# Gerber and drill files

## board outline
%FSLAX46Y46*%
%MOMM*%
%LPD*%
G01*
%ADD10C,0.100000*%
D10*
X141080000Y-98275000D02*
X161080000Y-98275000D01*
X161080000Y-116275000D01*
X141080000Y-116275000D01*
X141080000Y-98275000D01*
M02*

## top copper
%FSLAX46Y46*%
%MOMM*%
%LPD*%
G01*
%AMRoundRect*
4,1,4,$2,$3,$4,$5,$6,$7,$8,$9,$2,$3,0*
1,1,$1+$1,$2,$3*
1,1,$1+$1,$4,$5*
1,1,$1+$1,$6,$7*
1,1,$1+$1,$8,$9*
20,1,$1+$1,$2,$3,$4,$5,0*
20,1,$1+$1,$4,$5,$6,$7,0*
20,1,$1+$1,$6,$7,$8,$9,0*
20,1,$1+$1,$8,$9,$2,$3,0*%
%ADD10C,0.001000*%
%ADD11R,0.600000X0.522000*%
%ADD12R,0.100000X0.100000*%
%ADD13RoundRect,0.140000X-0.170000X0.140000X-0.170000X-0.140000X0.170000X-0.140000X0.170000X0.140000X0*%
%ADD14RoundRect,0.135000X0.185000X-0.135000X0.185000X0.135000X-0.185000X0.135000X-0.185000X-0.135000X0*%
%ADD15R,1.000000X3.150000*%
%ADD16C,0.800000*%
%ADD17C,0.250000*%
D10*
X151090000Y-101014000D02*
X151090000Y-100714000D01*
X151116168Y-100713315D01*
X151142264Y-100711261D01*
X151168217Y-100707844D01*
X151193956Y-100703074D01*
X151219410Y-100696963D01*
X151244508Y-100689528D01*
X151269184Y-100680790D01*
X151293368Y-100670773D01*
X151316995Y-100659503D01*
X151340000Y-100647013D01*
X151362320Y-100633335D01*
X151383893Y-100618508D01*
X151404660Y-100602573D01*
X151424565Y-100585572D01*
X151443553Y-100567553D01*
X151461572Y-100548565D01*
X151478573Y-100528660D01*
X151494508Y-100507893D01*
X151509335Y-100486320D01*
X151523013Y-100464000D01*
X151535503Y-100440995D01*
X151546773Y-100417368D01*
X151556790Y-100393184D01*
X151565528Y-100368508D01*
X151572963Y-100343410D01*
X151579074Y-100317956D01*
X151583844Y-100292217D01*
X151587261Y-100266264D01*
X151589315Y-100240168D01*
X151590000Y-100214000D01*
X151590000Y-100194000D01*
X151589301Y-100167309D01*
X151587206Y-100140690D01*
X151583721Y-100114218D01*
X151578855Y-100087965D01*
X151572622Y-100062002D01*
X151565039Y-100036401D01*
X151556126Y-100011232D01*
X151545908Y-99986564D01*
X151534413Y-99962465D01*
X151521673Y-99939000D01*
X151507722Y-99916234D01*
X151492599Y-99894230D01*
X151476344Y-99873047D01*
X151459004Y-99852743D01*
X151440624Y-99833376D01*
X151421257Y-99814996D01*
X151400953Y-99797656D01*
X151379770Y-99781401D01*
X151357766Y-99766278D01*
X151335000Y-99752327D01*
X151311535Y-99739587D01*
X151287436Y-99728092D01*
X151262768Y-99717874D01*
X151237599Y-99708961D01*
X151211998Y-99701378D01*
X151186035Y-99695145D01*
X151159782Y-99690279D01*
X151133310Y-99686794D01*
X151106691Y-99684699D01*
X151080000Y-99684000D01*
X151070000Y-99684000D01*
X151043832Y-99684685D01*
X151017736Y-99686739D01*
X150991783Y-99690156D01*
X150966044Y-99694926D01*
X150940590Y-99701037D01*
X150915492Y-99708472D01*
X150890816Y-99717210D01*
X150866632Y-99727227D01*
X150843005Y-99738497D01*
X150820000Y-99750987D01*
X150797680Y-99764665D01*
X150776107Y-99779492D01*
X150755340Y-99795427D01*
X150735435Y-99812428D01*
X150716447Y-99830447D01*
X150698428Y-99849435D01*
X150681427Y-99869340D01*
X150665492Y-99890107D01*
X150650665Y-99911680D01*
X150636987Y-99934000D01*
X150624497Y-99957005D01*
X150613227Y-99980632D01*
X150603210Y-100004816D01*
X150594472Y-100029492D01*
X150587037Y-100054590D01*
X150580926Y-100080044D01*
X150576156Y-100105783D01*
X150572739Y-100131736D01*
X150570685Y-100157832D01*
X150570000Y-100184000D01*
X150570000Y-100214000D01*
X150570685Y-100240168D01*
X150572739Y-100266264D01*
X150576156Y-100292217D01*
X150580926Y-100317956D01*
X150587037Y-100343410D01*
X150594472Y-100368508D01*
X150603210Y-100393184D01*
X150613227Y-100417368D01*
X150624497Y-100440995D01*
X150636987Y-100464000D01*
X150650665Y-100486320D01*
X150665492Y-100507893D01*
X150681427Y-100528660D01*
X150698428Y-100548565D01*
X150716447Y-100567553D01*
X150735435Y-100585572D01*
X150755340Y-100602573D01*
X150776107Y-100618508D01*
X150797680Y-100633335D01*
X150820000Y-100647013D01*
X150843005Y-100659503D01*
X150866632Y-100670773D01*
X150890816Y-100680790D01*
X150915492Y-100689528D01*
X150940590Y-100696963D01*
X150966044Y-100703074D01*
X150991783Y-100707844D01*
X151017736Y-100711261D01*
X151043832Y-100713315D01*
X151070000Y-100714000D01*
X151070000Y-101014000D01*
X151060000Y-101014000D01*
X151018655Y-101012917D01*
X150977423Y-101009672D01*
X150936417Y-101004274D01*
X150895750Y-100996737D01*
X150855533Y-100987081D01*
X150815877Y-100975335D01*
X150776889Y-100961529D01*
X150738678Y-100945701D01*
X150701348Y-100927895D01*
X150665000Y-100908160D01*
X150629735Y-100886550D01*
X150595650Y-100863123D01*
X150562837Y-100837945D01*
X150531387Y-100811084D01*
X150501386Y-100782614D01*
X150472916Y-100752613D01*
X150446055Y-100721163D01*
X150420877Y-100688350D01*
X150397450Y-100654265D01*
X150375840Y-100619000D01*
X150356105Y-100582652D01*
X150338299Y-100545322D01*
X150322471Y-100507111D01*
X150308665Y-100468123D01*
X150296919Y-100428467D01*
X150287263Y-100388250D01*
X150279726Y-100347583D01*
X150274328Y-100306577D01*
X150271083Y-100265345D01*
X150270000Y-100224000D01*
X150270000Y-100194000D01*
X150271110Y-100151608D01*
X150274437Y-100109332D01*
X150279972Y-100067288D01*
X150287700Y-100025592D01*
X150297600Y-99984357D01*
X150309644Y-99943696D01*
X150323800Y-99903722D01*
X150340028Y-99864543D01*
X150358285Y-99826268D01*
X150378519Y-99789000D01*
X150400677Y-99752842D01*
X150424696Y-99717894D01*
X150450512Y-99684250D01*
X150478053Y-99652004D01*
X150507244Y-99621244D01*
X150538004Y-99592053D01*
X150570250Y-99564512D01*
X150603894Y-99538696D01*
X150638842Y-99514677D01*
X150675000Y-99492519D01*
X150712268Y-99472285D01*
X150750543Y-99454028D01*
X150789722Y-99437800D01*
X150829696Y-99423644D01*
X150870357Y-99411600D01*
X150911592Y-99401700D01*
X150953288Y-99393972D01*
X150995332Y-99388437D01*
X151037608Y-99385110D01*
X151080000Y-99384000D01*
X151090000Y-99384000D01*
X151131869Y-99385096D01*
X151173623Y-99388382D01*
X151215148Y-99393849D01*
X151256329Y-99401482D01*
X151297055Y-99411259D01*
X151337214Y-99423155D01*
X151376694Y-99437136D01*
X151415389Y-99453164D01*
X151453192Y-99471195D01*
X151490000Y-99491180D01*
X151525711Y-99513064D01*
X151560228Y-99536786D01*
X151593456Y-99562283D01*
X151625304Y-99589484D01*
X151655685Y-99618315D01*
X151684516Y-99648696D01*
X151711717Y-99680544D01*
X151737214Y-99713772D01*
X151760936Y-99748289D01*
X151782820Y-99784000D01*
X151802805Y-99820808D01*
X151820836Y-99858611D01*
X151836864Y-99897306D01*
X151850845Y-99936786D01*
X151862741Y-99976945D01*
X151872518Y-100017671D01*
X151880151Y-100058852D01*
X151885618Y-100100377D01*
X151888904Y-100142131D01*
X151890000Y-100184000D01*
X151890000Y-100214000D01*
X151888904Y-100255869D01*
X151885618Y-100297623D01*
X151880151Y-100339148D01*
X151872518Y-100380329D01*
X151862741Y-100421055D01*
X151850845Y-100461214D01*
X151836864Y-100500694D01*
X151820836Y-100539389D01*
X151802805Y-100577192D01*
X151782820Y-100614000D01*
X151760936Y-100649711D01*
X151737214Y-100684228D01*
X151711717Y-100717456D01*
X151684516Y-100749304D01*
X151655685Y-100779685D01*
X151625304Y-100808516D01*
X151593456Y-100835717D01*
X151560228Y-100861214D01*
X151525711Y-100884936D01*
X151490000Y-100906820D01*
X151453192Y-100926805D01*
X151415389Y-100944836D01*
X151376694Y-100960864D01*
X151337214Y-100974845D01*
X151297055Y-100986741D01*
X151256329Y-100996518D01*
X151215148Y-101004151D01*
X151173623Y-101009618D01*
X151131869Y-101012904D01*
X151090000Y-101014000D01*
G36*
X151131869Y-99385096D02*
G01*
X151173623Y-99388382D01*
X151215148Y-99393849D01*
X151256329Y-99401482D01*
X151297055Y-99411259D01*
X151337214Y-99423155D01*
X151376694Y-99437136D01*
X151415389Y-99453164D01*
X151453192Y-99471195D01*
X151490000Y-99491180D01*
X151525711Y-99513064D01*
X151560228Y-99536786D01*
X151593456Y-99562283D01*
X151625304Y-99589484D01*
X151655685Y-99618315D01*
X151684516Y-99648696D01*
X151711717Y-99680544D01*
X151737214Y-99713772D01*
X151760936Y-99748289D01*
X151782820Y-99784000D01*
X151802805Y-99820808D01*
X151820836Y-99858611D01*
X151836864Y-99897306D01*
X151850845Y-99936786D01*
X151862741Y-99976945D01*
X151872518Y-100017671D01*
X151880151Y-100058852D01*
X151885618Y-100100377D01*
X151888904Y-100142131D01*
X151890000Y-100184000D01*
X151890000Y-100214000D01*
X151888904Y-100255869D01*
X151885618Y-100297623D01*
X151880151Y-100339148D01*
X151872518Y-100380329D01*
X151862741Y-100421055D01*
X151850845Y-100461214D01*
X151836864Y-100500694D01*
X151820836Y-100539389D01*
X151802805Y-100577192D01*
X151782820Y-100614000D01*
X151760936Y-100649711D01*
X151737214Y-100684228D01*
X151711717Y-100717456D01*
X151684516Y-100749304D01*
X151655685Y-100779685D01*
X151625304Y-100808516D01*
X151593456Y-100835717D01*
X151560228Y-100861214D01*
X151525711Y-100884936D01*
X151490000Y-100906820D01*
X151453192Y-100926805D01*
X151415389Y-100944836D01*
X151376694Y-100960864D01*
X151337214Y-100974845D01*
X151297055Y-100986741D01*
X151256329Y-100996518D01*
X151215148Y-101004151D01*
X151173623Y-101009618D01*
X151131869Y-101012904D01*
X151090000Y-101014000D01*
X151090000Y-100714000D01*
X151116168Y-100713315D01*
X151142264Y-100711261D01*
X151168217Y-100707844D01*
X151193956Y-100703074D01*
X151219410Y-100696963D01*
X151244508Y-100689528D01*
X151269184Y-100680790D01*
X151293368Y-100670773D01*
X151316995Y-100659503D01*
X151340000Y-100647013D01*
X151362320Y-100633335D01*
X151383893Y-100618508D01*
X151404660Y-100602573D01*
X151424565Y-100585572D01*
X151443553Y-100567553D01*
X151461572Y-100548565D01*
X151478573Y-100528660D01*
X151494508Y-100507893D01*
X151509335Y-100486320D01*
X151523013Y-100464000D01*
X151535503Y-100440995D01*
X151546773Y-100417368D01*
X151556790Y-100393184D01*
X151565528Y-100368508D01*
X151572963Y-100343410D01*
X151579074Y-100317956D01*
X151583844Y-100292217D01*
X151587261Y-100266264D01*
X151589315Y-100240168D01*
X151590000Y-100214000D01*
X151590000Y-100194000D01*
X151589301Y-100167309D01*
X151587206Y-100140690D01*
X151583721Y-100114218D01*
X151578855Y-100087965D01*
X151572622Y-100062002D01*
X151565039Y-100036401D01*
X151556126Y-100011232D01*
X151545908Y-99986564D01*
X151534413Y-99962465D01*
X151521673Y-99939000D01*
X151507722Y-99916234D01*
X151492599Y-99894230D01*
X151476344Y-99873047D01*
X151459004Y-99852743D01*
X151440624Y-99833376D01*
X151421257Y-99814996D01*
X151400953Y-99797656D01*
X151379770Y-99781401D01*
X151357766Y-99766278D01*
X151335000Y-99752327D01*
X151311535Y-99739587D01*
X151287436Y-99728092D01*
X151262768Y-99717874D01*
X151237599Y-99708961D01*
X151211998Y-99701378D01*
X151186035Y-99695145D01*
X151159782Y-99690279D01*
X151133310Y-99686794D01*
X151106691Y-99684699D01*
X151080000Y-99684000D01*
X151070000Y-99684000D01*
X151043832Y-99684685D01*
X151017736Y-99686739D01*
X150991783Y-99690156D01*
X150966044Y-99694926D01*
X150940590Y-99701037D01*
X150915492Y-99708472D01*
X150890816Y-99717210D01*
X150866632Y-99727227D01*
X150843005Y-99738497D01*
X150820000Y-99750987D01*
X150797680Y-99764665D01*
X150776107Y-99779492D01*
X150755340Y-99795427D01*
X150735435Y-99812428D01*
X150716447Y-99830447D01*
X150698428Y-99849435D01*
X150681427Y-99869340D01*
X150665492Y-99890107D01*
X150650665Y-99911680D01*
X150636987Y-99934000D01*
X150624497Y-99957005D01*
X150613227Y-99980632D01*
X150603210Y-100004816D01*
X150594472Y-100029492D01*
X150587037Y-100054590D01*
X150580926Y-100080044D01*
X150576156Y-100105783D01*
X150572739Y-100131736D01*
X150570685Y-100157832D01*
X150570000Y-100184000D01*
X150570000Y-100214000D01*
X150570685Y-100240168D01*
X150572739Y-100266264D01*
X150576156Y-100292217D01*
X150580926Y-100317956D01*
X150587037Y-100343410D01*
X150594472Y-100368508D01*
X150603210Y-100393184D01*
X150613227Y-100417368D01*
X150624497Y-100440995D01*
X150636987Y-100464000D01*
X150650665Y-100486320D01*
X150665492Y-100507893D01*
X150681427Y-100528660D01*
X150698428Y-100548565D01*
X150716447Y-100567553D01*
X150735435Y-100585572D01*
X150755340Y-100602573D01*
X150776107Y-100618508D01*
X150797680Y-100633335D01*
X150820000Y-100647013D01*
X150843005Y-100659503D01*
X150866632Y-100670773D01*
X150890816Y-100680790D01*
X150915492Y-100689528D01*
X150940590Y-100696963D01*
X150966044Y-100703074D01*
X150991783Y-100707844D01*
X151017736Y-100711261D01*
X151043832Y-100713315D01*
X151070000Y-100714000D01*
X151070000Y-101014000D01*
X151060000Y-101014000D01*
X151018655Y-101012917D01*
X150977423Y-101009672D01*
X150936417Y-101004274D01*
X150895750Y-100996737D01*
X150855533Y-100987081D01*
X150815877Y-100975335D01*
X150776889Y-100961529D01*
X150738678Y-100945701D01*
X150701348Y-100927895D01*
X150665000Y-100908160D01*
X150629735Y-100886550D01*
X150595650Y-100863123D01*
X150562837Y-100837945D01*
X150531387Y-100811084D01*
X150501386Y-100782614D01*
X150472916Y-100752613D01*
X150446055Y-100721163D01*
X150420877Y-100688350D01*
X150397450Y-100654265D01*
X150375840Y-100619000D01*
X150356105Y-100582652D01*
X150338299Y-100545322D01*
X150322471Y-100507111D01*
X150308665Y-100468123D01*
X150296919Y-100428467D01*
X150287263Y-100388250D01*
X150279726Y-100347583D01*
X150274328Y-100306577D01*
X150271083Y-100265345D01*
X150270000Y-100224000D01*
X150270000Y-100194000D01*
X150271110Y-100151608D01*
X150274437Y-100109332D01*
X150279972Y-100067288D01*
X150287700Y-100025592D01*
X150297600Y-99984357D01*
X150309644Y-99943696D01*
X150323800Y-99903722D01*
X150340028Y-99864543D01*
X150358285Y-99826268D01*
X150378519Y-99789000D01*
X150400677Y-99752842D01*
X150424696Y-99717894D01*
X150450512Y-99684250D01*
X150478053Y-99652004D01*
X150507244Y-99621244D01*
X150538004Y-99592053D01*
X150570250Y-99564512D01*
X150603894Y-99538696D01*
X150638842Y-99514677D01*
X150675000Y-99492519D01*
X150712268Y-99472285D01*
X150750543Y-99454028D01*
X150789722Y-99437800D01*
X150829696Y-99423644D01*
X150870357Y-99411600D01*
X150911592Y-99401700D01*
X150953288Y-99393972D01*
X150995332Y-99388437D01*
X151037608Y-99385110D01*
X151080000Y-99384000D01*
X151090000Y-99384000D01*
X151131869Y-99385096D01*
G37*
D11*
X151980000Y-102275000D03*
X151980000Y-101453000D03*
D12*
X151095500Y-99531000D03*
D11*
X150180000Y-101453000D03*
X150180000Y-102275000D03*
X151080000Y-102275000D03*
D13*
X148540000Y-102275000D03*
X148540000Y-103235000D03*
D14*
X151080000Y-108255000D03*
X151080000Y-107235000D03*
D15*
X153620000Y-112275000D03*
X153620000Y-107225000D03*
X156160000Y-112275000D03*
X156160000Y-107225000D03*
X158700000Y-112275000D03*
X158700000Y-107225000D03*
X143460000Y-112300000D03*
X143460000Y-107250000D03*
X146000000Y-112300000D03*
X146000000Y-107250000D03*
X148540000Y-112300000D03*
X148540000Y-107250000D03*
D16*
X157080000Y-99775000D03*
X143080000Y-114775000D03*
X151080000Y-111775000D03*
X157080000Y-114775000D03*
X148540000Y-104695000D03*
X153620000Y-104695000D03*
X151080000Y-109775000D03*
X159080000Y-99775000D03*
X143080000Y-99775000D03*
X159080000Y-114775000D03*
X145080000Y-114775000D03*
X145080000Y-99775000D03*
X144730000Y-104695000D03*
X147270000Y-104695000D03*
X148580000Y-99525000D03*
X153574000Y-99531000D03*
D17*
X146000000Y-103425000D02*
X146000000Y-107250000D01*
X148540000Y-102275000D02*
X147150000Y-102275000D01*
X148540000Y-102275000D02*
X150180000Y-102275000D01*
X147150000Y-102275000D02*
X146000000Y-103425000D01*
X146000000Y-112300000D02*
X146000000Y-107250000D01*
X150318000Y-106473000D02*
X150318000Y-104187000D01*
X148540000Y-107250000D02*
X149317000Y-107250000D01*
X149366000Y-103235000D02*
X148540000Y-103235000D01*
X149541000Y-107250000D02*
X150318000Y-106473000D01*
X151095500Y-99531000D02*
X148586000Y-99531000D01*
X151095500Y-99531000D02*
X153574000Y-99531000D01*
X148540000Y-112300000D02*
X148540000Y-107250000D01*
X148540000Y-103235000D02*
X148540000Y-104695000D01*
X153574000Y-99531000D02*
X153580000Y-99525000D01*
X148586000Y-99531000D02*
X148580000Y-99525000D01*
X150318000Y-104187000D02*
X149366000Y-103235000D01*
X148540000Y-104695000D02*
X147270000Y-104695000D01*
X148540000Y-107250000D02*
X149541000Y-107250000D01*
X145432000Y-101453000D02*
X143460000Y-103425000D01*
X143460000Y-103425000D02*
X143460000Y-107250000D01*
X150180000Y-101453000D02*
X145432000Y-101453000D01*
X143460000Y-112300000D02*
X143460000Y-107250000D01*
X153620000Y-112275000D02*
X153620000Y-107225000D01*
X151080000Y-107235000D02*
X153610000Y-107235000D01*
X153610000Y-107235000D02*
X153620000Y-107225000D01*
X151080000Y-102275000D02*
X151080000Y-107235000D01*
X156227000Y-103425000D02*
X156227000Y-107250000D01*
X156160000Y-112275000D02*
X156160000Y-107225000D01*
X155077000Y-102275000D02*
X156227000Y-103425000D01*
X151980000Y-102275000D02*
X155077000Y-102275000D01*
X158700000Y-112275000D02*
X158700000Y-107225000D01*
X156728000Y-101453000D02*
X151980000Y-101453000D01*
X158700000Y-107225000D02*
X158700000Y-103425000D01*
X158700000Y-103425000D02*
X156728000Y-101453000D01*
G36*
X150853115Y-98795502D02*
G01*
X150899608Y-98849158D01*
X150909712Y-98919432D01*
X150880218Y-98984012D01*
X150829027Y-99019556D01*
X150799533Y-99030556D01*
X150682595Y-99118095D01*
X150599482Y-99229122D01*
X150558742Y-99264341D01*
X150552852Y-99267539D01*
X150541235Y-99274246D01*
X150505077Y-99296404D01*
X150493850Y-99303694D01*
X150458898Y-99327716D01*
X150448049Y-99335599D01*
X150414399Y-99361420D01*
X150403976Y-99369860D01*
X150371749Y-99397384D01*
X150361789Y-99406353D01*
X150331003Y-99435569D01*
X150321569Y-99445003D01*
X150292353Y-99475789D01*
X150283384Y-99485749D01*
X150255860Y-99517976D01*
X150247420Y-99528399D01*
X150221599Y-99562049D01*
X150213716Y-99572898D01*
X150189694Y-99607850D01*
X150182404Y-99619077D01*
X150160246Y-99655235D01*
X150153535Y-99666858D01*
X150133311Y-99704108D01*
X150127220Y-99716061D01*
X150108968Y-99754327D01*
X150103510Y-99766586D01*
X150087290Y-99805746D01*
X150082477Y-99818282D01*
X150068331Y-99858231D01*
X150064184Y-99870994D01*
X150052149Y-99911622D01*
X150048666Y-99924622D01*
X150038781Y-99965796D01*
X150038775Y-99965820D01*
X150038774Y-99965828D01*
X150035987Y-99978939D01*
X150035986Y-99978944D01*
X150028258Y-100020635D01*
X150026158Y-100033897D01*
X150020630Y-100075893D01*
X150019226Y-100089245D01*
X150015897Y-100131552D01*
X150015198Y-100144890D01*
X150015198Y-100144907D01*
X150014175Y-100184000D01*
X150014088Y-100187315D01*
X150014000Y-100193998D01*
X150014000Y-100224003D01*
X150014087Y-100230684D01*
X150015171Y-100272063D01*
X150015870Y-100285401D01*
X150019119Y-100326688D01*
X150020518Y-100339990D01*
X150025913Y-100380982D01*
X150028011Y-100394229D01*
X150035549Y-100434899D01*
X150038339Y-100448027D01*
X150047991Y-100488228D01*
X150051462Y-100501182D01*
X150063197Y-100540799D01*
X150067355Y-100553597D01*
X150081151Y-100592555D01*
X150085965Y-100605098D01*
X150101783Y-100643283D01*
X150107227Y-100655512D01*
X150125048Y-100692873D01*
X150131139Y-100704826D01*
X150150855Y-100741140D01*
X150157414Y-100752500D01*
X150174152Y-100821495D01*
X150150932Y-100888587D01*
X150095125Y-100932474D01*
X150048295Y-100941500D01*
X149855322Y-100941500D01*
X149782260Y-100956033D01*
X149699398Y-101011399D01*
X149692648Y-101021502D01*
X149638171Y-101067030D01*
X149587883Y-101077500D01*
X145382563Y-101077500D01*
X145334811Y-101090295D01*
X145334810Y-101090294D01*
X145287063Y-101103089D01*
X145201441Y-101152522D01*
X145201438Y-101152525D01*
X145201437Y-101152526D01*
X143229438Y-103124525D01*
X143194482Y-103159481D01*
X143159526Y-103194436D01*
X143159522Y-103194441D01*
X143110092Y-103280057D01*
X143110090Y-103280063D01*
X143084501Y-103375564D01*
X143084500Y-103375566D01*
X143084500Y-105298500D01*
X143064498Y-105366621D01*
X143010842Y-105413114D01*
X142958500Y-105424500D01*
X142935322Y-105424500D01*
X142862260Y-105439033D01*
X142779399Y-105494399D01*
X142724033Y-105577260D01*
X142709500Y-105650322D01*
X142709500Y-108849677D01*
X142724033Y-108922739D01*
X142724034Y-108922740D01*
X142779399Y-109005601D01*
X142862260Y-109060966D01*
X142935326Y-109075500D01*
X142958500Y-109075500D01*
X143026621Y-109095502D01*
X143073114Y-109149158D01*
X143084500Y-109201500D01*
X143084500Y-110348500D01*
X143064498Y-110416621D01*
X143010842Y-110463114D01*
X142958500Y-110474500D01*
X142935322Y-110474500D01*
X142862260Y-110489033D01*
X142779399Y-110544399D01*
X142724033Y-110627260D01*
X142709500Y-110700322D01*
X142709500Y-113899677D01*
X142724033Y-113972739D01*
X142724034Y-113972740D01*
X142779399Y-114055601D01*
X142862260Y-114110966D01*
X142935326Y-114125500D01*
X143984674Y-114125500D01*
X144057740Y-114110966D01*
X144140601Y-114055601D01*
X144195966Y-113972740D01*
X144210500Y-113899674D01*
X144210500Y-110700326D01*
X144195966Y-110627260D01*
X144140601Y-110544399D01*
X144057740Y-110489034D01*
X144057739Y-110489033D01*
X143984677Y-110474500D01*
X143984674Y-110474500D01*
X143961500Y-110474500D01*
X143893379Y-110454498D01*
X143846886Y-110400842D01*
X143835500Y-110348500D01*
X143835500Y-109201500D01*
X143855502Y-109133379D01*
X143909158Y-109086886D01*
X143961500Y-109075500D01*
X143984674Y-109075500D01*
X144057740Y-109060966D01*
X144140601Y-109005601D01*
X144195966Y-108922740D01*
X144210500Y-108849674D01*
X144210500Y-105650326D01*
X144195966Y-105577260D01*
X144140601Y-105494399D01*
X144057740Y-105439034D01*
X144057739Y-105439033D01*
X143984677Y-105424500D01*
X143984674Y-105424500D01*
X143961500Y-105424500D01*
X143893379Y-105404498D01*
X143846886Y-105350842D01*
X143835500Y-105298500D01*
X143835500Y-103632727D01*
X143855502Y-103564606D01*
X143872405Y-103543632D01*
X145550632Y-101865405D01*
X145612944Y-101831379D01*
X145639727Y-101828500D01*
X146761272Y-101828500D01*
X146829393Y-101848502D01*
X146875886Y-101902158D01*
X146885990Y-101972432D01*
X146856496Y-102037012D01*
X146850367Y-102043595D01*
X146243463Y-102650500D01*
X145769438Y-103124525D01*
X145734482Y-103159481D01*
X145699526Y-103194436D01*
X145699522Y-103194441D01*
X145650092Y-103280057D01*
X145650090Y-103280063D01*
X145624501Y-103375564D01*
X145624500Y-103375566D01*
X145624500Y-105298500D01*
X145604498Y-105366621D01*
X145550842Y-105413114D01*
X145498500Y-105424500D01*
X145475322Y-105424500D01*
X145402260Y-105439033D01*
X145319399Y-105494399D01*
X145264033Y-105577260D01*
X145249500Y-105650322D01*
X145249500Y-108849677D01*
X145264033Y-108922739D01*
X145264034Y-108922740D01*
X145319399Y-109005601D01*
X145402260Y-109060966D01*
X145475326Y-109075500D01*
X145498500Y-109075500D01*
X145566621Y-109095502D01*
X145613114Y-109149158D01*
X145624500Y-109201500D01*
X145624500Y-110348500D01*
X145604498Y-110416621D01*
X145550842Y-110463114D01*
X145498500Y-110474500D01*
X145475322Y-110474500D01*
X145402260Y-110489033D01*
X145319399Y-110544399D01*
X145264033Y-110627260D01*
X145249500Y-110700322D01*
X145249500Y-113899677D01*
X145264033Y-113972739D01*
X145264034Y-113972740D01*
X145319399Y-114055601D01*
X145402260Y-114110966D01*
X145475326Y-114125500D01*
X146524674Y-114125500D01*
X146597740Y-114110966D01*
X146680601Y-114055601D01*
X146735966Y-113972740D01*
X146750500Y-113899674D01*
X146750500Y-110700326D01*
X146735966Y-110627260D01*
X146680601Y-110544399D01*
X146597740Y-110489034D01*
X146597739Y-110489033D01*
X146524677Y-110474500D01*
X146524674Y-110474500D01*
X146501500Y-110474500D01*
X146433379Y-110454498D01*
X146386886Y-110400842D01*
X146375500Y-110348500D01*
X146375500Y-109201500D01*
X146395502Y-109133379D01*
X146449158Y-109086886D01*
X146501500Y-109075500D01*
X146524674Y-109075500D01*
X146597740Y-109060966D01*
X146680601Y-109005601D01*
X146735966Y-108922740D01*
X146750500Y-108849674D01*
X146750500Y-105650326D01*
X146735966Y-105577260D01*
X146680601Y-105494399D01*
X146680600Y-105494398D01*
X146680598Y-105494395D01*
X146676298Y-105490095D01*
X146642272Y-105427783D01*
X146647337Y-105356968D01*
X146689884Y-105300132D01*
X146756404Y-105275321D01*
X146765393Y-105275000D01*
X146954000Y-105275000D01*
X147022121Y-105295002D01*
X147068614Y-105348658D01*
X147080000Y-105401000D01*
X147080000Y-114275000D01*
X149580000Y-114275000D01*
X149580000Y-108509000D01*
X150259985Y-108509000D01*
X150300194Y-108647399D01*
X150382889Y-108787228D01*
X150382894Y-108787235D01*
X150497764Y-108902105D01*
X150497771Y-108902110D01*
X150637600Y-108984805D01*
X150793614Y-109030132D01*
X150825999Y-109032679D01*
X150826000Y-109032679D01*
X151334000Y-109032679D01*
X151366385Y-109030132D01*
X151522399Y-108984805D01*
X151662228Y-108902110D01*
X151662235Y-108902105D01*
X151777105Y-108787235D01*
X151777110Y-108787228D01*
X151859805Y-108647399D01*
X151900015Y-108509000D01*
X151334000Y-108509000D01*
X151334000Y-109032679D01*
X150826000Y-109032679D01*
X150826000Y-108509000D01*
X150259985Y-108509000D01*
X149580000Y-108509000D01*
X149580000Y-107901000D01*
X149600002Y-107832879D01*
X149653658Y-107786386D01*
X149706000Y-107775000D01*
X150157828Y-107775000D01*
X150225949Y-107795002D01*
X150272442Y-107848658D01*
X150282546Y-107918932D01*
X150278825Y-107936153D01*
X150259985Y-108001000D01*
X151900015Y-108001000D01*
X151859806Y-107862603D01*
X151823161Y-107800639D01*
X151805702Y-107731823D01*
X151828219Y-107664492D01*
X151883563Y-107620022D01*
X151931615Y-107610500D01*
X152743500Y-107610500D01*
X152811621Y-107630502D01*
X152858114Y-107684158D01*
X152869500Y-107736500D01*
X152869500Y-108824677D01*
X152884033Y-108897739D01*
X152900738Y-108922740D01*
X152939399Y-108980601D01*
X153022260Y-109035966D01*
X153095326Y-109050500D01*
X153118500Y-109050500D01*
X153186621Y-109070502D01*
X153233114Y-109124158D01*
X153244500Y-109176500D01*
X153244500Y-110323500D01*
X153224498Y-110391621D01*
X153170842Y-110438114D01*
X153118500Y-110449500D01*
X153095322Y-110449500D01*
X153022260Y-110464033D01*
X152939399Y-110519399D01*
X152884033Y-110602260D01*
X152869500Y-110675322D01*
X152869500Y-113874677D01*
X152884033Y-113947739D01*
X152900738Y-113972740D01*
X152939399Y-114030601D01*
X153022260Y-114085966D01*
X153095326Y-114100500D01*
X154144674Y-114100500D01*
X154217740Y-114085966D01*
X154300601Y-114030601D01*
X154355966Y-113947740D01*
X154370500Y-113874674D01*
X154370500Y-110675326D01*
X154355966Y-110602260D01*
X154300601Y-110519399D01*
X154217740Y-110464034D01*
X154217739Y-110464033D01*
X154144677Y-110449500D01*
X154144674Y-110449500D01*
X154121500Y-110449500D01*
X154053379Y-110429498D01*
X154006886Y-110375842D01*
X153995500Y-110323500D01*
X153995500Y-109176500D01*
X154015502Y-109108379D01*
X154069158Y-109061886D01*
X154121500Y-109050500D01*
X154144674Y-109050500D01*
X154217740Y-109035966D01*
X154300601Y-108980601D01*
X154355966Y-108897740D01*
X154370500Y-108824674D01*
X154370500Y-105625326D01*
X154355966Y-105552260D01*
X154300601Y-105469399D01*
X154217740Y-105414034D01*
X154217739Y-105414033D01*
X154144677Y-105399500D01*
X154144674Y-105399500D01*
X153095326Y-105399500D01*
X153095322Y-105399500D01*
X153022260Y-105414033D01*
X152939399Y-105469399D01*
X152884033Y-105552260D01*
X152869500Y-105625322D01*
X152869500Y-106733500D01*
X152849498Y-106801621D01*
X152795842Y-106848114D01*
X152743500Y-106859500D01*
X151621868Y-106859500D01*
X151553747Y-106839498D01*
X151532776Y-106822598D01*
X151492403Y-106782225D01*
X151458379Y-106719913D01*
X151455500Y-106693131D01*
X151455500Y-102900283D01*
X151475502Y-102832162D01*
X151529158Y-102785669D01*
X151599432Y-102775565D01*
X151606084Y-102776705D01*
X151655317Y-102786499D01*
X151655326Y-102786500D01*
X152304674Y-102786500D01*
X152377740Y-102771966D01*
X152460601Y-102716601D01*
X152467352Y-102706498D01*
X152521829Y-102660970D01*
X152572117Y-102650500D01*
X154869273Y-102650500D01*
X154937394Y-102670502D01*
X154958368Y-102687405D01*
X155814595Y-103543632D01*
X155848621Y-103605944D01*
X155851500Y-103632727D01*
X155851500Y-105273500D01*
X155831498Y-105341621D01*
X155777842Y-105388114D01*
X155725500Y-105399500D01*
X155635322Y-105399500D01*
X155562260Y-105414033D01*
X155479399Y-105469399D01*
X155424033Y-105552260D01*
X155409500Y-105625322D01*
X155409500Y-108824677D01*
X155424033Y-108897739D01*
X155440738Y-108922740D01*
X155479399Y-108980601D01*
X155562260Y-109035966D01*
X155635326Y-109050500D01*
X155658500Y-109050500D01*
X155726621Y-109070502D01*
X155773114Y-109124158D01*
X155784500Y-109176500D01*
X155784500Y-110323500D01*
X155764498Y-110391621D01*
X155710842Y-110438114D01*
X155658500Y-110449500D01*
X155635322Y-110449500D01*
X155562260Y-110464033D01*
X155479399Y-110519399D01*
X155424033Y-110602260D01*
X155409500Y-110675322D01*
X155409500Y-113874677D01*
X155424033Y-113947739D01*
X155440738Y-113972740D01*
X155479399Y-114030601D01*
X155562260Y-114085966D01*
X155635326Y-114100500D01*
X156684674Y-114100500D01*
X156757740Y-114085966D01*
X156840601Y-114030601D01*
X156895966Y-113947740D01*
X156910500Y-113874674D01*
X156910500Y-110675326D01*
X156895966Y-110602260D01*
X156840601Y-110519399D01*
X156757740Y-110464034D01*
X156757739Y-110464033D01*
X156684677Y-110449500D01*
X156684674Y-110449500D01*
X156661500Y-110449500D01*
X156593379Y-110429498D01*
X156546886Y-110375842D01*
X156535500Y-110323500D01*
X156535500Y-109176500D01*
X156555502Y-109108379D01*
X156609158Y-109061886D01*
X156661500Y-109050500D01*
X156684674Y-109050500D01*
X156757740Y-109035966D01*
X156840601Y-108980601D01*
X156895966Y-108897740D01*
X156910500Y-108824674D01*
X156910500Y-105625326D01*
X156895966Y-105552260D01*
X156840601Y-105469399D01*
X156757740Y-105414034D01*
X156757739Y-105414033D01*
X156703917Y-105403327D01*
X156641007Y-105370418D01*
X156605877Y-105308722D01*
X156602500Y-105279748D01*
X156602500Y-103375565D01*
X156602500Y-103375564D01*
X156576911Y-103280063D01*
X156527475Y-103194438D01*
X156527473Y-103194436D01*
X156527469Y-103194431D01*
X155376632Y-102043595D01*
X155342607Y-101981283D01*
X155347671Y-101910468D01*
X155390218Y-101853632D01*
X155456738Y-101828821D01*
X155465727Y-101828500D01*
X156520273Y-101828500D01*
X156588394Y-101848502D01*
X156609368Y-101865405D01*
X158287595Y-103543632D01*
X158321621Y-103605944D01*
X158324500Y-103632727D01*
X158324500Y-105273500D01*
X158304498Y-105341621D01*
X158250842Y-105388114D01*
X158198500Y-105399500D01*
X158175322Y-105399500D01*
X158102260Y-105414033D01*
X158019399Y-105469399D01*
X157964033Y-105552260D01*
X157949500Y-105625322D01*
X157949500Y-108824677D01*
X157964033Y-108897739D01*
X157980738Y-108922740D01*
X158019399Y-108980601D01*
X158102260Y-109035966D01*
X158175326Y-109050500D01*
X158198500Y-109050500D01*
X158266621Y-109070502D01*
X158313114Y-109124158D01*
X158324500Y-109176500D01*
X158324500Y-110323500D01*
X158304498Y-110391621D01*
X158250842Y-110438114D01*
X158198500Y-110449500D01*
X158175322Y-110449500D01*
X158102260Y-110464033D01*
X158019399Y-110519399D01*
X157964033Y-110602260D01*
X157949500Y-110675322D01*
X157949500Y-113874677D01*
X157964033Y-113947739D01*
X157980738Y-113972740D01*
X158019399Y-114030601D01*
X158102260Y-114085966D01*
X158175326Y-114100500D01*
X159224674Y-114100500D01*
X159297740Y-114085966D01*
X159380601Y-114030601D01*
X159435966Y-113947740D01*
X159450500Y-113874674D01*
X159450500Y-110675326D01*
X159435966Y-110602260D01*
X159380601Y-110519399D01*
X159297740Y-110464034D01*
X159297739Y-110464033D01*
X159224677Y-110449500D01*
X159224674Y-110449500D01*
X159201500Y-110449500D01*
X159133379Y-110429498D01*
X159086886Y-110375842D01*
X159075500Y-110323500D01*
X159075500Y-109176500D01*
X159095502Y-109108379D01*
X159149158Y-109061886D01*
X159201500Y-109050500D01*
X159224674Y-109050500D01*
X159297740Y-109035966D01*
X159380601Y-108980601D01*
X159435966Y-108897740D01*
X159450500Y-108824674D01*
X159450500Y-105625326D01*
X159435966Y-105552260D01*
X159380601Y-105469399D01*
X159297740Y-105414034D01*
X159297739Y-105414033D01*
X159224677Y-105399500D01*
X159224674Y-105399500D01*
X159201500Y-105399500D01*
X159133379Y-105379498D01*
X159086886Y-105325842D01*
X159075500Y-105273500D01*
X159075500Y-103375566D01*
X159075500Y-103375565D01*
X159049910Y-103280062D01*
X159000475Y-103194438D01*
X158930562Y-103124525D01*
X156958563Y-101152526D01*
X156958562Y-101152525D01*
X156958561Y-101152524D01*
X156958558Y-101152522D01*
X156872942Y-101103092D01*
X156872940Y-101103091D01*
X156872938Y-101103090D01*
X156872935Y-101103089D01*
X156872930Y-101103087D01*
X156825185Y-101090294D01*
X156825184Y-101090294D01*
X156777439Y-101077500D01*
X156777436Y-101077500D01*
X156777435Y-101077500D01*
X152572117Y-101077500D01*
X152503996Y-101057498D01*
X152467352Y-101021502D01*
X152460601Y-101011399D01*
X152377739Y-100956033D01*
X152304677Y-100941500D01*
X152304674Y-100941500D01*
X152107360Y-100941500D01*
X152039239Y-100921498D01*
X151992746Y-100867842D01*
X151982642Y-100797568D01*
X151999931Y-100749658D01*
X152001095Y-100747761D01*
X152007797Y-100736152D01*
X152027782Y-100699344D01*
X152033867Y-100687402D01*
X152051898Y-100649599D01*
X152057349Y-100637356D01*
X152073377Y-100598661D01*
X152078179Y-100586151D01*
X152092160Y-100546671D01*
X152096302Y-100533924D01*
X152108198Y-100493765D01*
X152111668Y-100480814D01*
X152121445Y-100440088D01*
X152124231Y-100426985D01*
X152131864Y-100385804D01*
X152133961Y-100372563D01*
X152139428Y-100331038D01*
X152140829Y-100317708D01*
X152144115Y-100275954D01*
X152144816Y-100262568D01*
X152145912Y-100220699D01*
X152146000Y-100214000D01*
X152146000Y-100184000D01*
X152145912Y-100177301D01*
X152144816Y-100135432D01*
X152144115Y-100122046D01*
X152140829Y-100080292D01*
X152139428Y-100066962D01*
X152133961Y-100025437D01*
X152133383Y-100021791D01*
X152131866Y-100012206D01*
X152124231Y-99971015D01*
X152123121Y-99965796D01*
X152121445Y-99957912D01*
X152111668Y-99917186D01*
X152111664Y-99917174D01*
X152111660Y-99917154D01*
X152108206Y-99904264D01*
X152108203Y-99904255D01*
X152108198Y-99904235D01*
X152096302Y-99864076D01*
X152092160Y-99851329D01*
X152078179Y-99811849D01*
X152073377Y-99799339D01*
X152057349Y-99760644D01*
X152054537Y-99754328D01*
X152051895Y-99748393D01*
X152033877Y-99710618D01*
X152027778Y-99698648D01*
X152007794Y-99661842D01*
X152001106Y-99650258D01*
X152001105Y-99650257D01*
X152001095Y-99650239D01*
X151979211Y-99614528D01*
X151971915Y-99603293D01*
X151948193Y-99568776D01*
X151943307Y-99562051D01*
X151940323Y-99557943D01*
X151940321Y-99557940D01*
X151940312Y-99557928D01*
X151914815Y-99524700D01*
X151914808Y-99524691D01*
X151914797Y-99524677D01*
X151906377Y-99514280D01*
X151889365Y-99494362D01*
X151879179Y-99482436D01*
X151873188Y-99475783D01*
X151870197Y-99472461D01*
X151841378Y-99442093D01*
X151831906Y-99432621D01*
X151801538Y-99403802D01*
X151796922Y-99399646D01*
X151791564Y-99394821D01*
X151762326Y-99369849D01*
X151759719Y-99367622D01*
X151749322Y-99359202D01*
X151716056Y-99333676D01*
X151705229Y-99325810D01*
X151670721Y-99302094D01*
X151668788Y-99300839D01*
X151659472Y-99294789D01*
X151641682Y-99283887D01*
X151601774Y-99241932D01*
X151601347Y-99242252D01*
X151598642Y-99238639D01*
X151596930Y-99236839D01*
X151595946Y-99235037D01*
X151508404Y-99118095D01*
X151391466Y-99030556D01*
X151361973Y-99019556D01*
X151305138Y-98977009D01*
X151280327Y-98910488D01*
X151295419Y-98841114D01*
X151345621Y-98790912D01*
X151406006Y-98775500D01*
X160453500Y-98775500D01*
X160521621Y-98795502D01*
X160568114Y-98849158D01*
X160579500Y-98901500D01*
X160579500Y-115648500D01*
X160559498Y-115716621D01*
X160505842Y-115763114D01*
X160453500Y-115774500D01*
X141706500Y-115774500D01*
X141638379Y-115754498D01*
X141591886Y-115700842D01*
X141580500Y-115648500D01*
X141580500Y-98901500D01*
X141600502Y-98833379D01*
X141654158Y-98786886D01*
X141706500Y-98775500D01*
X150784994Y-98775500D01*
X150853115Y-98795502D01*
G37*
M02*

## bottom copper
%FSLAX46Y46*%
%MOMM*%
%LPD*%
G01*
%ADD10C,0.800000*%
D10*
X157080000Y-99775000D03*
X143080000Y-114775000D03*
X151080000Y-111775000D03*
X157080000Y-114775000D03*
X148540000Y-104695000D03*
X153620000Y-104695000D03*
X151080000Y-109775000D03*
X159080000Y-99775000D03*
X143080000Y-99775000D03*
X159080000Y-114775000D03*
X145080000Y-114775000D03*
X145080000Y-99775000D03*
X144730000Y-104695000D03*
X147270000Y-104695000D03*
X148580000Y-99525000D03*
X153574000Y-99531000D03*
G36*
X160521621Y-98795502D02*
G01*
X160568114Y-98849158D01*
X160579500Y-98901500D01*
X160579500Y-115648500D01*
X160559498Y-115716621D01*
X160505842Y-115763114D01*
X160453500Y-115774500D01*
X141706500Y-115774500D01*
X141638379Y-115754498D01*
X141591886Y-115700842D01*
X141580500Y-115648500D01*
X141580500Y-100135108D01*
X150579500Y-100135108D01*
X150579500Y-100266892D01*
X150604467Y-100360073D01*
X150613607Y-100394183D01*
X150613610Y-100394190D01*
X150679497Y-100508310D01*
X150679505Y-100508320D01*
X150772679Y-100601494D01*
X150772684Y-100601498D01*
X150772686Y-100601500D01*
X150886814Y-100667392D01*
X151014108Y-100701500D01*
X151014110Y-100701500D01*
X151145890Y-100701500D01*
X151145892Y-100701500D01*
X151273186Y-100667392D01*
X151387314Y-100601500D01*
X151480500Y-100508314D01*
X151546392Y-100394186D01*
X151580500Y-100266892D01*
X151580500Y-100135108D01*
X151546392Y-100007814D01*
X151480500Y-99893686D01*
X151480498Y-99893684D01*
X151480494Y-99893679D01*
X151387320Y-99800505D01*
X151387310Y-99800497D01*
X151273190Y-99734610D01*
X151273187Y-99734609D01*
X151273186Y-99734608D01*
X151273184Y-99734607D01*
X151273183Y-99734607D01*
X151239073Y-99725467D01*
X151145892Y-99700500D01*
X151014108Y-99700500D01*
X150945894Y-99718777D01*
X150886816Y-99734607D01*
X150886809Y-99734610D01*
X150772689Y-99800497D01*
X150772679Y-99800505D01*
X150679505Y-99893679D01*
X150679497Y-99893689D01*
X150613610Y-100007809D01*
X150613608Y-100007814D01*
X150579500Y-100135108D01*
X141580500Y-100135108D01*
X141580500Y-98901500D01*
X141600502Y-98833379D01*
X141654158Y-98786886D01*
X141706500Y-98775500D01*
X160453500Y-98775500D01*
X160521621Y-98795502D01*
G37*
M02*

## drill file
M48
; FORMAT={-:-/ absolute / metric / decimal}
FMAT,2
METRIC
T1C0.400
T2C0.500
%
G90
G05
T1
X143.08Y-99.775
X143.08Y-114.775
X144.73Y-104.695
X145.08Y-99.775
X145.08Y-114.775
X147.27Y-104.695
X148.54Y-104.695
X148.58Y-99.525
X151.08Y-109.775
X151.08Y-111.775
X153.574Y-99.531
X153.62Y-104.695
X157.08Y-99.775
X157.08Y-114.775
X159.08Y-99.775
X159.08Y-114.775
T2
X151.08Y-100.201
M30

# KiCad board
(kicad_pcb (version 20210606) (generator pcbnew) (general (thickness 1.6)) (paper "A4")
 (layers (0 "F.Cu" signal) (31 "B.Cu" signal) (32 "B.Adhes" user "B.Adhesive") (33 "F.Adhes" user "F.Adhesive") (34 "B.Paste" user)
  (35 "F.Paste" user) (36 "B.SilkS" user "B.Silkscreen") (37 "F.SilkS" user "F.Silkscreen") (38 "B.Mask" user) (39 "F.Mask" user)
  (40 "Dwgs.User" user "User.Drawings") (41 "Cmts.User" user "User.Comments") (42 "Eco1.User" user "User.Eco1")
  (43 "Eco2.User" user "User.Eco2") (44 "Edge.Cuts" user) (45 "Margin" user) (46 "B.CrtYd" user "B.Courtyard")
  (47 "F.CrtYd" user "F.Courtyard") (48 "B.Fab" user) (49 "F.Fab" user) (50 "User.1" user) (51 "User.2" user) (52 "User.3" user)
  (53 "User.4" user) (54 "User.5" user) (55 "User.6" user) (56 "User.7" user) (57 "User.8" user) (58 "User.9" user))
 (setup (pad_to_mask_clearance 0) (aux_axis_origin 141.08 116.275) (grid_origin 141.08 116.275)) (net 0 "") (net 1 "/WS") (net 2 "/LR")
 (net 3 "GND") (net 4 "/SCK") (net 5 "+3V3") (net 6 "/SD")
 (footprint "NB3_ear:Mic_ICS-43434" (layer "F.Cu") (at 151.08 100.914 180)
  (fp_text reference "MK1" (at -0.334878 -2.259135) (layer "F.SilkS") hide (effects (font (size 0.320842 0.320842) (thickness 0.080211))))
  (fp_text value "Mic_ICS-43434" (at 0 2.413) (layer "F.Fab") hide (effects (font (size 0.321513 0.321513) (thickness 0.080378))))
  (fp_poly
   (pts (xy -0.01 -0.1) (xy -0.01 0.2) (xy -0.036168 0.200685) (xy -0.062264 0.202739) (xy -0.088217 0.206156) (xy -0.113956 0.210926)
    (xy -0.13941 0.217037) (xy -0.164508 0.224472) (xy -0.189184 0.23321) (xy -0.213368 0.243227) (xy -0.236995 0.254497)
    (xy -0.26 0.266987) (xy -0.28232 0.280665) (xy -0.303893 0.295492) (xy -0.32466 0.311427) (xy -0.344565 0.328428)
    (xy -0.363553 0.346447) (xy -0.381572 0.365435) (xy -0.398573 0.38534) (xy -0.414508 0.406107) (xy -0.429335 0.42768)
    (xy -0.443013 0.45) (xy -0.455503 0.473005) (xy -0.466773 0.496632) (xy -0.47679 0.520816) (xy -0.485528 0.545492)
    (xy -0.492963 0.57059) (xy -0.499074 0.596044) (xy -0.503844 0.621783) (xy -0.507261 0.647736) (xy -0.509315 0.673832) (xy -0.51 0.7)
    (xy -0.51 0.72) (xy -0.509301 0.746691) (xy -0.507206 0.77331) (xy -0.503721 0.799782) (xy -0.498855 0.826035) (xy -0.492622 0.851998)
    (xy -0.485039 0.877599) (xy -0.476126 0.902768) (xy -0.465908 0.927436) (xy -0.454413 0.951535) (xy -0.441673 0.975)
    (xy -0.427722 0.997766) (xy -0.412599 1.01977) (xy -0.396344 1.040953) (xy -0.379004 1.061257) (xy -0.360624 1.080624)
    (xy -0.341257 1.099004) (xy -0.320953 1.116344) (xy -0.29977 1.132599) (xy -0.277766 1.147722) (xy -0.255 1.161673)
    (xy -0.231535 1.174413) (xy -0.207436 1.185908) (xy -0.182768 1.196126) (xy -0.157599 1.205039) (xy -0.131998 1.212622)
    (xy -0.106035 1.218855) (xy -0.079782 1.223721) (xy -0.05331 1.227206) (xy -0.026691 1.229301) (xy 0 1.23) (xy 0.01 1.23)
    (xy 0.036168 1.229315) (xy 0.062264 1.227261) (xy 0.088217 1.223844) (xy 0.113956 1.219074) (xy 0.13941 1.212963) (xy 0.164508 1.205528)
    (xy 0.189184 1.19679) (xy 0.213368 1.186773) (xy 0.236995 1.175503) (xy 0.26 1.163013) (xy 0.28232 1.149335) (xy 0.303893 1.134508)
    (xy 0.32466 1.118573) (xy 0.344565 1.101572) (xy 0.363553 1.083553) (xy 0.381572 1.064565) (xy 0.398573 1.04466) (xy 0.414508 1.023893)
    (xy 0.429335 1.00232) (xy 0.443013 0.98) (xy 0.455503 0.956995) (xy 0.466773 0.933368) (xy 0.47679 0.909184) (xy 0.485528 0.884508)
    (xy 0.492963 0.85941) (xy 0.499074 0.833956) (xy 0.503844 0.808217) (xy 0.507261 0.782264) (xy 0.509315 0.756168) (xy 0.51 0.73)
    (xy 0.51 0.7) (xy 0.509315 0.673832) (xy 0.507261 0.647736) (xy 0.503844 0.621783) (xy 0.499074 0.596044) (xy 0.492963 0.57059)
    (xy 0.485528 0.545492) (xy 0.47679 0.520816) (xy 0.466773 0.496632) (xy 0.455503 0.473005) (xy 0.443013 0.45) (xy 0.429335 0.42768)
    (xy 0.414508 0.406107) (xy 0.398573 0.38534) (xy 0.381572 0.365435) (xy 0.363553 0.346447) (xy 0.344565 0.328428) (xy 0.32466 0.311427)
    (xy 0.303893 0.295492) (xy 0.28232 0.280665) (xy 0.26 0.266987) (xy 0.236995 0.254497) (xy 0.213368 0.243227) (xy 0.189184 0.23321)
    (xy 0.164508 0.224472) (xy 0.13941 0.217037) (xy 0.113956 0.210926) (xy 0.088217 0.206156) (xy 0.062264 0.202739) (xy 0.036168 0.200685)
    (xy 0.01 0.2) (xy 0.01 -0.1) (xy 0.02 -0.1) (xy 0.061345 -0.098917) (xy 0.102577 -0.095672) (xy 0.143583 -0.090274)
    (xy 0.18425 -0.082737) (xy 0.224467 -0.073081) (xy 0.264123 -0.061335) (xy 0.303111 -0.047529) (xy 0.341322 -0.031701)
    (xy 0.378652 -0.013895) (xy 0.415 0.00584) (xy 0.450265 0.02745) (xy 0.48435 0.050877) (xy 0.517163 0.076055) (xy 0.548613 0.102916)
    (xy 0.578614 0.131386) (xy 0.607084 0.161387) (xy 0.633945 0.192837) (xy 0.659123 0.22565) (xy 0.68255 0.259735) (xy 0.70416 0.295)
    (xy 0.723895 0.331348) (xy 0.741701 0.368678) (xy 0.757529 0.406889) (xy 0.771335 0.445877) (xy 0.783081 0.485533) (xy 0.792737 0.52575)
    (xy 0.800274 0.566417) (xy 0.805672 0.607423) (xy 0.808917 0.648655) (xy 0.81 0.69) (xy 0.81 0.72) (xy 0.80889 0.762392)
    (xy 0.805563 0.804668) (xy 0.800028 0.846712) (xy 0.7923 0.888408) (xy 0.7824 0.929643) (xy 0.770356 0.970304) (xy 0.7562 1.010278)
    (xy 0.739972 1.049457) (xy 0.721715 1.087732) (xy 0.701481 1.125) (xy 0.679323 1.161158) (xy 0.655304 1.196106) (xy 0.629488 1.22975)
    (xy 0.601947 1.261996) (xy 0.572756 1.292756) (xy 0.541996 1.321947) (xy 0.50975 1.349488) (xy 0.476106 1.375304) (xy 0.441158 1.399323)
    (xy 0.405 1.421481) (xy 0.367732 1.441715) (xy 0.329457 1.459972) (xy 0.290278 1.4762) (xy 0.250304 1.490356) (xy 0.209643 1.5024)
    (xy 0.168408 1.5123) (xy 0.126712 1.520028) (xy 0.084668 1.525563) (xy 0.042392 1.52889) (xy 0 1.53) (xy -0.01 1.53)
    (xy -0.051869 1.528904) (xy -0.093623 1.525618) (xy -0.135148 1.520151) (xy -0.176329 1.512518) (xy -0.217055 1.502741)
    (xy -0.257214 1.490845) (xy -0.296694 1.476864) (xy -0.335389 1.460836) (xy -0.373192 1.442805) (xy -0.41 1.42282)
    (xy -0.445711 1.400936) (xy -0.480228 1.377214) (xy -0.513456 1.351717) (xy -0.545304 1.324516) (xy -0.575685 1.295685)
    (xy -0.604516 1.265304) (xy -0.631717 1.233456) (xy -0.657214 1.200228) (xy -0.680936 1.165711) (xy -0.70282 1.13)
    (xy -0.722805 1.093192) (xy -0.740836 1.055389) (xy -0.756864 1.016694) (xy -0.770845 0.977214) (xy -0.782741 0.937055)
    (xy -0.792518 0.896329) (xy -0.800151 0.855148) (xy -0.805618 0.813623) (xy -0.808904 0.771869) (xy -0.81 0.73) (xy -0.81 0.7)
    (xy -0.808904 0.658131) (xy -0.805618 0.616377) (xy -0.800151 0.574852) (xy -0.792518 0.533671) (xy -0.782741 0.492945)
    (xy -0.770845 0.452786) (xy -0.756864 0.413306) (xy -0.740836 0.374611) (xy -0.722805 0.336808) (xy -0.70282 0.3)
    (xy -0.680936 0.264289) (xy -0.657214 0.229772) (xy -0.631717 0.196544) (xy -0.604516 0.164696) (xy -0.575685 0.134315)
    (xy -0.545304 0.105484) (xy -0.513456 0.078283) (xy -0.480228 0.052786) (xy -0.445711 0.029064) (xy -0.41 0.00718)
    (xy -0.373192 -0.012805) (xy -0.335389 -0.030836) (xy -0.296694 -0.046864) (xy -0.257214 -0.060845) (xy -0.217055 -0.072741)
    (xy -0.176329 -0.082518) (xy -0.135148 -0.090151) (xy -0.093623 -0.095618) (xy -0.051869 -0.098904) (xy -0.01 -0.1))
   (layer "F.Cu") (width 0.001) (fill solid))
  (pad "1" smd rect locked (at -0.9 -1.361 180) (size 0.6 0.522) (layers "F.Cu" "F.Mask") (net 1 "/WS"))
  (pad "2" smd rect locked (at -0.9 -0.539 180) (size 0.6 0.522) (layers "F.Cu" "F.Mask") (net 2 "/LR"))
  (pad "3" smd rect locked (at -0.0155 1.383 180) (size 0.1 0.1) (layers "F.Cu") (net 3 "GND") (zone_connect 1))
  (pad "4" smd rect locked (at 0.9 -0.539 180) (size 0.6 0.522) (layers "F.Cu" "F.Mask") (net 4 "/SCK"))
  (pad "5" smd rect locked (at 0.9 -1.361 180) (size 0.6 0.522) (layers "F.Cu" "F.Mask") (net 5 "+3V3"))
  (pad "6" smd rect locked (at 0 -1.361 180) (size 0.6 0.522) (layers "F.Cu" "F.Mask") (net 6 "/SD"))
  (pad "None" np_thru_hole circle locked (at 0 0.713 180) (size 0.5 0.5) (drill 0.5) (layers *.Cu *.Mask)))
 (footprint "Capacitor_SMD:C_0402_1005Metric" (layer "F.Cu") (at 148.54 102.755 -90)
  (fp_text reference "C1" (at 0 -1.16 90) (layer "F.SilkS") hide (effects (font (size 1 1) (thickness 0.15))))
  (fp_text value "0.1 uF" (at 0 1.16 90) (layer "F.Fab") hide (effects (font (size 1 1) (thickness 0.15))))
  (pad "1" smd roundrect locked (at -0.48 0 270) (size 0.56 0.62) (layers "F.Cu" "F.Paste" "F.Mask") (roundrect_rratio 0.25) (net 5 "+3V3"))
  (pad "2" smd roundrect locked (at 0.48 0 270) (size 0.56 0.62) (layers "F.Cu" "F.Paste" "F.Mask") (roundrect_rratio 0.25) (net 3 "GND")))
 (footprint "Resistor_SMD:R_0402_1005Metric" (layer "F.Cu") (at 151.08 107.745 90)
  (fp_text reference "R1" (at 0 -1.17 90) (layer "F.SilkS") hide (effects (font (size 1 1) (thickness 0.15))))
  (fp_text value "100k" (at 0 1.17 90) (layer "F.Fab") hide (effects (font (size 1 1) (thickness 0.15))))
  (pad "1" smd roundrect locked (at -0.51 0 90) (size 0.54 0.64) (layers "F.Cu" "F.Paste" "F.Mask") (roundrect_rratio 0.25) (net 3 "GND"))
  (pad "2" smd roundrect locked (at 0.51 0 90) (size 0.54 0.64) (layers "F.Cu" "F.Paste" "F.Mask") (roundrect_rratio 0.25) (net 6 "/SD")))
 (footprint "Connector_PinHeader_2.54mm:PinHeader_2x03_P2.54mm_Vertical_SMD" (layer "F.Cu") (at 156.16 109.75 90)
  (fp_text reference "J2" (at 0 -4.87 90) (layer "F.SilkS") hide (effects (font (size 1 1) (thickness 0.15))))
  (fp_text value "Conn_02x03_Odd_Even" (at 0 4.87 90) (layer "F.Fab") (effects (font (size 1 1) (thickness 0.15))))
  (pad "1" smd rect locked (at -2.525 -2.54 90) (size 3.15 1) (layers "F.Cu" "F.Paste" "F.Mask") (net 6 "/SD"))
  (pad "2" smd rect locked (at 2.525 -2.54 90) (size 3.15 1) (layers "F.Cu" "F.Paste" "F.Mask") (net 6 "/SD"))
  (pad "3" smd rect locked (at -2.525 0 90) (size 3.15 1) (layers "F.Cu" "F.Paste" "F.Mask") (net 1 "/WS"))
  (pad "4" smd rect locked (at 2.525 0 90) (size 3.15 1) (layers "F.Cu" "F.Paste" "F.Mask") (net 1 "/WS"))
  (pad "5" smd rect locked (at -2.525 2.54 90) (size 3.15 1) (layers "F.Cu" "F.Paste" "F.Mask") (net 2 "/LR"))
  (pad "6" smd rect locked (at 2.525 2.54 90) (size 3.15 1) (layers "F.Cu" "F.Paste" "F.Mask") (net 2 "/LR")))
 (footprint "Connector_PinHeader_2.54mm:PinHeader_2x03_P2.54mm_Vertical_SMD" (layer "F.Cu") (at 146 109.775 90)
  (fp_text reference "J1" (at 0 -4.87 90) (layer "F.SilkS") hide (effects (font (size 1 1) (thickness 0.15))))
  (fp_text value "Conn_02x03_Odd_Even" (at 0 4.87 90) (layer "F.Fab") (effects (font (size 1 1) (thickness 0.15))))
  (pad "1" smd rect locked (at -2.525 -2.54 90) (size 3.15 1) (layers "F.Cu" "F.Paste" "F.Mask") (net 4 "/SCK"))
  (pad "2" smd rect locked (at 2.525 -2.54 90) (size 3.15 1) (layers "F.Cu" "F.Paste" "F.Mask") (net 4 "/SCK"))
  (pad "3" smd rect locked (at -2.525 0 90) (size 3.15 1) (layers "F.Cu" "F.Paste" "F.Mask") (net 5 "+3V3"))
  (pad "4" smd rect locked (at 2.525 0 90) (size 3.15 1) (layers "F.Cu" "F.Paste" "F.Mask") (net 5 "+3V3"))
  (pad "5" smd rect locked (at -2.525 2.54 90) (size 3.15 1) (layers "F.Cu" "F.Paste" "F.Mask") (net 3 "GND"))
  (pad "6" smd rect locked (at 2.525 2.54 90) (size 3.15 1) (layers "F.Cu" "F.Paste" "F.Mask") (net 3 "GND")))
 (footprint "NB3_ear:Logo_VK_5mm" (layer "B.Cu") (at 151.08 107.275 180)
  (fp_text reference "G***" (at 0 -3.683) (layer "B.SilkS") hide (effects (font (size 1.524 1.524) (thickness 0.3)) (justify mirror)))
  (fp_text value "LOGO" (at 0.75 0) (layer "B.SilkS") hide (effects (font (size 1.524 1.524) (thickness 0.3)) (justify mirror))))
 (gr_rect (start 141.08 116.275) (end 161.08 98.275) (layer "Edge.Cuts") (width 0.1) (fill none))
 (segment (start 146 103.425) (end 146 107.25) (width 0.25) (layer "F.Cu") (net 5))
 (segment (start 148.54 102.275) (end 147.15 102.275) (width 0.25) (layer "F.Cu") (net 5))
 (segment (start 148.54 102.275) (end 150.18 102.275) (width 0.25) (layer "F.Cu") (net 5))
 (segment (start 147.15 102.275) (end 146 103.425) (width 0.25) (layer "F.Cu") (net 5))
 (segment (start 146 112.3) (end 146 107.25) (width 0.25) (layer "F.Cu") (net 5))
 (segment (start 150.318 106.473) (end 150.318 104.187) (width 0.25) (layer "F.Cu") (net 3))
 (segment (start 148.54 107.25) (end 149.317 107.25) (width 0.25) (layer "F.Cu") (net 3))
 (segment (start 149.366 103.235) (end 148.54 103.235) (width 0.25) (layer "F.Cu") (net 3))
 (segment (start 149.541 107.25) (end 150.318 106.473) (width 0.25) (layer "F.Cu") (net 3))
 (segment (start 151.0955 99.531) (end 148.586 99.531) (width 0.25) (layer "F.Cu") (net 3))
 (segment (start 151.0955 99.531) (end 153.574 99.531) (width 0.25) (layer "F.Cu") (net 3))
 (segment (start 148.54 112.3) (end 148.54 107.25) (width 0.25) (layer "F.Cu") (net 3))
 (segment (start 148.54 103.235) (end 148.54 104.695) (width 0.25) (layer "F.Cu") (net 3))
 (segment (start 153.574 99.531) (end 153.58 99.525) (width 0.25) (layer "F.Cu") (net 3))
 (segment (start 148.586 99.531) (end 148.58 99.525) (width 0.25) (layer "F.Cu") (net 3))
 (segment (start 150.318 104.187) (end 149.366 103.235) (width 0.25) (layer "F.Cu") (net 3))
 (segment (start 148.54 104.695) (end 147.27 104.695) (width 0.25) (layer "F.Cu") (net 3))
 (segment (start 148.54 107.25) (end 149.541 107.25) (width 0.25) (layer "F.Cu") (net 3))
 (via (at 157.08 99.775) (size 0.8) (drill 0.4) (layers "F.Cu" "B.Cu") (free) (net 3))
 (via (at 143.08 114.775) (size 0.8) (drill 0.4) (layers "F.Cu" "B.Cu") (free) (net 3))
 (via (at 151.08 111.775) (size 0.8) (drill 0.4) (layers "F.Cu" "B.Cu") (free) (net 3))
 (via (at 157.08 114.775) (size 0.8) (drill 0.4) (layers "F.Cu" "B.Cu") (free) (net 3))
 (via (at 148.54 104.695) (size 0.8) (drill 0.4) (layers "F.Cu" "B.Cu") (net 3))
 (via (at 153.62 104.695) (size 0.8) (drill 0.4) (layers "F.Cu" "B.Cu") (free) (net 3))
 (via (at 151.08 109.775) (size 0.8) (drill 0.4) (layers "F.Cu" "B.Cu") (free) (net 3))
 (via (at 159.08 99.775) (size 0.8) (drill 0.4) (layers "F.Cu" "B.Cu") (free) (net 3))
 (via (at 143.08 99.775) (size 0.8) (drill 0.4) (layers "F.Cu" "B.Cu") (free) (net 3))
 (via (at 159.08 114.775) (size 0.8) (drill 0.4) (layers "F.Cu" "B.Cu") (free) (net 3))
 (via (at 145.08 114.775) (size 0.8) (drill 0.4) (layers "F.Cu" "B.Cu") (free) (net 3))
 (via (at 145.08 99.775) (size 0.8) (drill 0.4) (layers "F.Cu" "B.Cu") (free) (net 3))
 (via (at 144.73 104.695) (size 0.8) (drill 0.4) (layers "F.Cu" "B.Cu") (free) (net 3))
 (via (at 147.27 104.695) (size 0.8) (drill 0.4) (layers "F.Cu" "B.Cu") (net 3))
 (via (at 148.58 99.525) (size 0.8) (drill 0.4) (layers "F.Cu" "B.Cu") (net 3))
 (via (at 153.574 99.531) (size 0.8) (drill 0.4) (layers "F.Cu" "B.Cu") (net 3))
 (segment (start 145.432 101.453) (end 143.46 103.425) (width 0.25) (layer "F.Cu") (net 4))
 (segment (start 143.46 103.425) (end 143.46 107.25) (width 0.25) (layer "F.Cu") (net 4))
 (segment (start 150.18 101.453) (end 145.432 101.453) (width 0.25) (layer "F.Cu") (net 4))
 (segment (start 143.46 112.3) (end 143.46 107.25) (width 0.25) (layer "F.Cu") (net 4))
 (segment (start 153.62 112.275) (end 153.62 107.225) (width 0.25) (layer "F.Cu") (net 6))
 (segment (start 151.08 107.235) (end 153.61 107.235) (width 0.25) (layer "F.Cu") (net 6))
 (segment (start 153.61 107.235) (end 153.62 107.225) (width 0.25) (layer "F.Cu") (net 6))
 (segment (start 151.08 102.275) (end 151.08 107.235) (width 0.25) (layer "F.Cu") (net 6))
 (segment (start 156.227 103.425) (end 156.227 107.25) (width 0.25) (layer "F.Cu") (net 1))
 (segment (start 156.16 112.275) (end 156.16 107.225) (width 0.25) (layer "F.Cu") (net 1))
 (segment (start 155.077 102.275) (end 156.227 103.425) (width 0.25) (layer "F.Cu") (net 1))
 (segment (start 151.98 102.275) (end 155.077 102.275) (width 0.25) (layer "F.Cu") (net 1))
 (segment (start 158.7 112.275) (end 158.7 107.225) (width 0.25) (layer "F.Cu") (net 2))
 (segment (start 156.728 101.453) (end 151.98 101.453) (width 0.25) (layer "F.Cu") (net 2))
 (segment (start 158.7 107.225) (end 158.7 103.425) (width 0.25) (layer "F.Cu") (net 2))
 (segment (start 158.7 103.425) (end 156.728 101.453) (width 0.25) (layer "F.Cu") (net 2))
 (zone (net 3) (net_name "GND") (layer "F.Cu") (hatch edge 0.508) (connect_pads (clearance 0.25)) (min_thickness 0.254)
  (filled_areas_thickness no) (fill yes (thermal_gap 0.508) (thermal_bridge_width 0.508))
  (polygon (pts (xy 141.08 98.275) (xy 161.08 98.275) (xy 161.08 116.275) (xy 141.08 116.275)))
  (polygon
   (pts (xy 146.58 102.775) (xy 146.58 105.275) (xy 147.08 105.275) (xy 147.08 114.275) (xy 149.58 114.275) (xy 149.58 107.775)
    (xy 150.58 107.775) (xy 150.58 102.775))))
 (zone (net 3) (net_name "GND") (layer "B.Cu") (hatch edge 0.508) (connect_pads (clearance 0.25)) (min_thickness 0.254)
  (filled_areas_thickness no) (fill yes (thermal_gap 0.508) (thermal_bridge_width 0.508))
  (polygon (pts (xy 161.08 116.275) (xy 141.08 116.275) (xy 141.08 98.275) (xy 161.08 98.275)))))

